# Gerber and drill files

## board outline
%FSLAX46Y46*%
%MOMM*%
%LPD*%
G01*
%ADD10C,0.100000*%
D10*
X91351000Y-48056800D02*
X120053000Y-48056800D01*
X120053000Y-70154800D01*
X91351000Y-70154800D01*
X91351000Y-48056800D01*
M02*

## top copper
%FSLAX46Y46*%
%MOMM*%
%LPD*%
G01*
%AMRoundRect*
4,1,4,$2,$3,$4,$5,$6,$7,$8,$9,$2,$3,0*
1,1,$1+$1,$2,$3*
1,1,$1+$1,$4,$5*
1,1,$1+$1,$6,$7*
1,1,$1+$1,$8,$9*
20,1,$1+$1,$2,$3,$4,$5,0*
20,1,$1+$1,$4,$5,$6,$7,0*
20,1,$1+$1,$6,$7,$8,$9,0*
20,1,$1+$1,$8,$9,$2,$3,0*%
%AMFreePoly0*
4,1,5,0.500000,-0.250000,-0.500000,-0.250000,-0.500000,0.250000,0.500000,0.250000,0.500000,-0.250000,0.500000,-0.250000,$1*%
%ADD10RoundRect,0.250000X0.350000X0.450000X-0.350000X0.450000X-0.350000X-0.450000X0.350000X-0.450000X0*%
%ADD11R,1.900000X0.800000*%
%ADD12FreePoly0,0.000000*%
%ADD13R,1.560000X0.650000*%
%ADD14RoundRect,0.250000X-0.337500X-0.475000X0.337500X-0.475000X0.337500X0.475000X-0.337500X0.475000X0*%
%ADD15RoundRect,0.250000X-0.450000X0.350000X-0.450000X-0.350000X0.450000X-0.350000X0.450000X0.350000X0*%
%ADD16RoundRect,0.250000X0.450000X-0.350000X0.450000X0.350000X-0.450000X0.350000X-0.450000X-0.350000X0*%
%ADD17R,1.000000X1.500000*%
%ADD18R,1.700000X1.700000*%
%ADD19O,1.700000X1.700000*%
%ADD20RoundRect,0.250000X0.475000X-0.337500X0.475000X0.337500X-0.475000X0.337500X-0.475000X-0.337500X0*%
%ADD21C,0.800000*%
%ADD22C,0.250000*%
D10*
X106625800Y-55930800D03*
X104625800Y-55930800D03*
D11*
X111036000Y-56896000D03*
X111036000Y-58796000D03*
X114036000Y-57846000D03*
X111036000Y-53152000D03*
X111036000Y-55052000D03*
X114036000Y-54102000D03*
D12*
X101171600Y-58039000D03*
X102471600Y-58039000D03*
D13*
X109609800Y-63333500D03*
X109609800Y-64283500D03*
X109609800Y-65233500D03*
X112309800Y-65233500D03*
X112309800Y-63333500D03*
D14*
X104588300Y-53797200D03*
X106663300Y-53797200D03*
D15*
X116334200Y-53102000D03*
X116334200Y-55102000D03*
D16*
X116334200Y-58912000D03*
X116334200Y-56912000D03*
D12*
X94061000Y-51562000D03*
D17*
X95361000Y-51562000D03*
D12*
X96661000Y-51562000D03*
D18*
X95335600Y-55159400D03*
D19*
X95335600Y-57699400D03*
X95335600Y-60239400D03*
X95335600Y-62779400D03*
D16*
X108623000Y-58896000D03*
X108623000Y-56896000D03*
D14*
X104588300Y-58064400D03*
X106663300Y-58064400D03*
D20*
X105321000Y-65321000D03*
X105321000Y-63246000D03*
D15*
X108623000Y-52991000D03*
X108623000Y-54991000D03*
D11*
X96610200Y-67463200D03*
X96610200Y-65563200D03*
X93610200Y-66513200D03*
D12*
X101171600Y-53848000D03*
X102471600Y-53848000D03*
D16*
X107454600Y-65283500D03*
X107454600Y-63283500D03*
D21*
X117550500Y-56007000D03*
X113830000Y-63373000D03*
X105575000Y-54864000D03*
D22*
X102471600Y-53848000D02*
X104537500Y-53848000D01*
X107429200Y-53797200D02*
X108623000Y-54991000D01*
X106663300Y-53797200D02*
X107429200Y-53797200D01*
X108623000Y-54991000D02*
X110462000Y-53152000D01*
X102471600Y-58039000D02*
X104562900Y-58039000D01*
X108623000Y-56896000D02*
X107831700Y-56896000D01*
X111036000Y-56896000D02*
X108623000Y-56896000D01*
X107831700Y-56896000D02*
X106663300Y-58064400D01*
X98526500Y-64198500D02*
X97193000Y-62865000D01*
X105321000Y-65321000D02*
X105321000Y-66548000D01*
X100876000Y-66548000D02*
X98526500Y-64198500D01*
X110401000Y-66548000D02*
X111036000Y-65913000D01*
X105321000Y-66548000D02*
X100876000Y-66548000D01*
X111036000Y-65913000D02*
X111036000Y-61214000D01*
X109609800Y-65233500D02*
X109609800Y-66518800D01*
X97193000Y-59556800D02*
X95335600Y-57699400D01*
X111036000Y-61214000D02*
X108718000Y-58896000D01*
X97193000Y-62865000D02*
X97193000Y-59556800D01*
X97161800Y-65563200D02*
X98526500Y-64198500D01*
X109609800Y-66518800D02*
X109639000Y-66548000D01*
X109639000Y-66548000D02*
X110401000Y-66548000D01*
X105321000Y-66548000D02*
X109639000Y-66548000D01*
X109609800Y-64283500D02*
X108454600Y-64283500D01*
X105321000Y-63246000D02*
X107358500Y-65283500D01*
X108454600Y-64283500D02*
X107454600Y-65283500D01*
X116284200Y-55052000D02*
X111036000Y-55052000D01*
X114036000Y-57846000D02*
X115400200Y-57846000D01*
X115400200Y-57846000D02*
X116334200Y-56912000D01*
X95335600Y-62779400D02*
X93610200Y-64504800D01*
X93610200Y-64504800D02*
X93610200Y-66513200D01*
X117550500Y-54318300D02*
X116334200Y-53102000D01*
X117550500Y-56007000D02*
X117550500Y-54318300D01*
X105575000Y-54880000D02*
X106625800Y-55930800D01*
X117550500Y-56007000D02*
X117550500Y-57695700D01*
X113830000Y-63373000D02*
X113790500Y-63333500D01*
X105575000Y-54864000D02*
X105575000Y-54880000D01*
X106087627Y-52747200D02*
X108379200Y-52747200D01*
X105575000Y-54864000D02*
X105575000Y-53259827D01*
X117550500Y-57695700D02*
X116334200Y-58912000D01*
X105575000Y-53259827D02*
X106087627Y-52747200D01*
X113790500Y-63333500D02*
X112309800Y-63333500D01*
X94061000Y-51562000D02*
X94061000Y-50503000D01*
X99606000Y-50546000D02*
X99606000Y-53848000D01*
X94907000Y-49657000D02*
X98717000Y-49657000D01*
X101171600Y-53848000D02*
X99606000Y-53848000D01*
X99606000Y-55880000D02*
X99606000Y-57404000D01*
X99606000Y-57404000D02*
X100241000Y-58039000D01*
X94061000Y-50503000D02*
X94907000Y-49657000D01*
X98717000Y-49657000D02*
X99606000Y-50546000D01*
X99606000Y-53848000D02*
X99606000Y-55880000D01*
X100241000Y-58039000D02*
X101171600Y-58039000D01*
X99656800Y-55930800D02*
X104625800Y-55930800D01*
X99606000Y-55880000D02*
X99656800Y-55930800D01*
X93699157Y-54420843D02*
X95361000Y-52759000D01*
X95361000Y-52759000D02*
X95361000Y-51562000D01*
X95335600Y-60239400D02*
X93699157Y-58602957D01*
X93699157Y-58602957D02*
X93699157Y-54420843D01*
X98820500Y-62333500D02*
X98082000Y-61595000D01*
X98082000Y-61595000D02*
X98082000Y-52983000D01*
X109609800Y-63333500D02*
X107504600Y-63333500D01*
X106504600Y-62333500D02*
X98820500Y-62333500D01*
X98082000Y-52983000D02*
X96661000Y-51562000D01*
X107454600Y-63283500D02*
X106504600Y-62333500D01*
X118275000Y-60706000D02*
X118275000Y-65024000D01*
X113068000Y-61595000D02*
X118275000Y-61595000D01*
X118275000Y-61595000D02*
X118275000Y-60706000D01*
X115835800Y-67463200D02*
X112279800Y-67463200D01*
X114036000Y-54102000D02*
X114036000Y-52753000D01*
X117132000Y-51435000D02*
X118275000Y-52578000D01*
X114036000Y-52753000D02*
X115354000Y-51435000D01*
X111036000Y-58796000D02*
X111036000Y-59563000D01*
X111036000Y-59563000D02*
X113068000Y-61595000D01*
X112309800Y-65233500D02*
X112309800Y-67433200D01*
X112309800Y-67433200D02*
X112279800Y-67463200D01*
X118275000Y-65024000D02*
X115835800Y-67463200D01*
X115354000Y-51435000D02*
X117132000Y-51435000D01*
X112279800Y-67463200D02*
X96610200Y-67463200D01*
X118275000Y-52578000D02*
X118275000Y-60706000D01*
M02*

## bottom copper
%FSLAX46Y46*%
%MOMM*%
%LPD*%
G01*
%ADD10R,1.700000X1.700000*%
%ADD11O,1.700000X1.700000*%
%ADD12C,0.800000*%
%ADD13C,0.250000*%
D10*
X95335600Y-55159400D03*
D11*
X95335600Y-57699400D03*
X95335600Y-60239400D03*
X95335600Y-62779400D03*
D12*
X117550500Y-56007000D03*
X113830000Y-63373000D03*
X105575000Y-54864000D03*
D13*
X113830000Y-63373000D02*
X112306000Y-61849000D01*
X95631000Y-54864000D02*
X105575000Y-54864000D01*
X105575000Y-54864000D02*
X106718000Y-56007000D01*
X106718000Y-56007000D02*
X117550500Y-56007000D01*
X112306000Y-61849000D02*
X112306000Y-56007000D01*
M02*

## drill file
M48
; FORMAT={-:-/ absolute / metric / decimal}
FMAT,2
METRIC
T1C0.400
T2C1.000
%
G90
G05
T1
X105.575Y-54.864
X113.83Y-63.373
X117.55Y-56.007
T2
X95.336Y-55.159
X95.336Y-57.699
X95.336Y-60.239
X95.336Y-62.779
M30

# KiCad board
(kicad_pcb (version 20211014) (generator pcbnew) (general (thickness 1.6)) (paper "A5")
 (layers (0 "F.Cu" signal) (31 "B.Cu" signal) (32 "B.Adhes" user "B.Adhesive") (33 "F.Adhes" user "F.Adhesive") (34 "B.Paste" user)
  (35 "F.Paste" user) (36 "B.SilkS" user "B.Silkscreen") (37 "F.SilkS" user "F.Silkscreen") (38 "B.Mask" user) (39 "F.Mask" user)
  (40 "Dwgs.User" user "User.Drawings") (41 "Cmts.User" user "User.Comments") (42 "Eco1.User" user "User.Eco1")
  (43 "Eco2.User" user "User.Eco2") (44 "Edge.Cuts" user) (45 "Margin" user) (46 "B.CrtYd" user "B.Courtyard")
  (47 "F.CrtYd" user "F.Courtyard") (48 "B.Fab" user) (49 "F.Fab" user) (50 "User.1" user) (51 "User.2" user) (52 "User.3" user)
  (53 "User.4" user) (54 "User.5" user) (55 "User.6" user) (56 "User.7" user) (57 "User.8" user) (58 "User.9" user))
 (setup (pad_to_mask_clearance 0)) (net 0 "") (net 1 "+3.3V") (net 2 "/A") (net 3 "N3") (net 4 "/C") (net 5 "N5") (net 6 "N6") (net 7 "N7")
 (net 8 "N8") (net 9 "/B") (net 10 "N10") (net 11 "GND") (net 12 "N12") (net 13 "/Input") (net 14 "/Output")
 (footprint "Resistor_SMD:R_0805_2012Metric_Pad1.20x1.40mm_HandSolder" (layer "F.Cu") (at 105.6258 55.9308 180)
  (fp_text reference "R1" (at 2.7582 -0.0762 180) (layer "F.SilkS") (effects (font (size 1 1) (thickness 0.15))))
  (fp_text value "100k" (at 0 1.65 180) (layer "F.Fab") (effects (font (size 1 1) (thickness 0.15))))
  (pad "1" smd roundrect (at -1 0 180) (size 1.2 1.4) (layers "F.Cu" "F.Paste" "F.Mask") (roundrect_rratio 0.2083333333) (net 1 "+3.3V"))
  (pad "2" smd roundrect (at 1 0 180) (size 1.2 1.4) (layers "F.Cu" "F.Paste" "F.Mask") (roundrect_rratio 0.2083333333) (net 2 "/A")))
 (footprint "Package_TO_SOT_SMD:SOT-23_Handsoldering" (layer "F.Cu") (at 112.536 57.846)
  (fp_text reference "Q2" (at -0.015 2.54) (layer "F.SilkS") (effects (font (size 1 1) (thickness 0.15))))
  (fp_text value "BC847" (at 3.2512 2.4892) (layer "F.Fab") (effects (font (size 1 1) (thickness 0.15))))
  (pad "1" smd rect (at -1.5 -0.95) (size 1.9 0.8) (layers "F.Cu" "F.Paste" "F.Mask") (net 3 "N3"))
  (pad "2" smd rect (at -1.5 0.95) (size 1.9 0.8) (layers "F.Cu" "F.Paste" "F.Mask") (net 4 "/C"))
  (pad "3" smd rect (at 1.5 0) (size 1.9 0.8) (layers "F.Cu" "F.Paste" "F.Mask") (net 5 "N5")))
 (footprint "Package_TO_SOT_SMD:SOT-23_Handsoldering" (layer "F.Cu") (at 112.536 54.102)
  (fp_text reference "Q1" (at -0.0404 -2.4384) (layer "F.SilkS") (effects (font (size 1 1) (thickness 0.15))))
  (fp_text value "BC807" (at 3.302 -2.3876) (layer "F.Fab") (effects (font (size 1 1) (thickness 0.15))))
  (pad "1" smd rect (at -1.5 -0.95) (size 1.9 0.8) (layers "F.Cu" "F.Paste" "F.Mask") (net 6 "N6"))
  (pad "2" smd rect (at -1.5 0.95) (size 1.9 0.8) (layers "F.Cu" "F.Paste" "F.Mask") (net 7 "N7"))
  (pad "3" smd rect (at 1.5 0) (size 1.9 0.8) (layers "F.Cu" "F.Paste" "F.Mask") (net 4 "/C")))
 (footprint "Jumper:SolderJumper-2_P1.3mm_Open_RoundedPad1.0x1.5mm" (layer "F.Cu") (at 101.8216 58.039)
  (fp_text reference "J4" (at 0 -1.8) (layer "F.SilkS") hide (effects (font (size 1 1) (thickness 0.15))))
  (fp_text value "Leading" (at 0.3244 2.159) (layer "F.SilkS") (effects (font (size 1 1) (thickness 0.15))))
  (pad "1" smd custom (at -0.65 0) (size 1 0.5) (layers "F.Cu" "F.Mask") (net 2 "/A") (zone_connect 2)
   (options (clearance outline) (anchor rect)) (primitives))
  (pad "2" smd custom (at 0.65 0) (size 1 0.5) (layers "F.Cu" "F.Mask") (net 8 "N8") (zone_connect 2)
   (options (clearance outline) (anchor rect)) (primitives)))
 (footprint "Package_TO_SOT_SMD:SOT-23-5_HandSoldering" (layer "F.Cu") (at 110.9598 64.2835)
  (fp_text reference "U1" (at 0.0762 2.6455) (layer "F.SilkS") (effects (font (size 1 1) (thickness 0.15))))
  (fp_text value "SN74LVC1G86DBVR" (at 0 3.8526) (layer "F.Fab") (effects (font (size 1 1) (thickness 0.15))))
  (pad "1" smd rect (at -1.35 -0.95) (size 1.56 0.65) (layers "F.Cu" "F.Paste" "F.Mask") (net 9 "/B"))
  (pad "2" smd rect (at -1.35 0) (size 1.56 0.65) (layers "F.Cu" "F.Paste" "F.Mask") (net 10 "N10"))
  (pad "3" smd rect (at -1.35 0.95) (size 1.56 0.65) (layers "F.Cu" "F.Paste" "F.Mask") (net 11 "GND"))
  (pad "4" smd rect (at 1.35 0.95) (size 1.56 0.65) (layers "F.Cu" "F.Paste" "F.Mask") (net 4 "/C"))
  (pad "5" smd rect (at 1.35 -0.95) (size 1.56 0.65) (layers "F.Cu" "F.Paste" "F.Mask") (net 1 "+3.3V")))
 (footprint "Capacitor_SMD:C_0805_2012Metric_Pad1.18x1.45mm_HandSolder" (layer "F.Cu") (at 105.6258 53.7972)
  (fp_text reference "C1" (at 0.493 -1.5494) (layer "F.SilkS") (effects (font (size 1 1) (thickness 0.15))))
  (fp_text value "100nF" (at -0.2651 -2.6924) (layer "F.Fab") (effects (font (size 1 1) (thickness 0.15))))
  (pad "1" smd roundrect (at -1.0375 0) (size 1.175 1.45) (layers "F.Cu" "F.Paste" "F.Mask") (roundrect_rratio 0.2127659574) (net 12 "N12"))
  (pad "2" smd roundrect (at 1.0375 0) (size 1.175 1.45) (layers "F.Cu" "F.Paste" "F.Mask") (roundrect_rratio 0.2127659574) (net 6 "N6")))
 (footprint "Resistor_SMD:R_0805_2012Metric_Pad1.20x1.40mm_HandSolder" (layer "F.Cu") (at 116.3342 54.102 -90)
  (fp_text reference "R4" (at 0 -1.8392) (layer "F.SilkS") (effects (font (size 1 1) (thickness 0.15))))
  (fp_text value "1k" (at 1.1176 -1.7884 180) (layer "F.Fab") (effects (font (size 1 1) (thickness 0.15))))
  (pad "1" smd roundrect (at -1 0 270) (size 1.2 1.4) (layers "F.Cu" "F.Paste" "F.Mask") (roundrect_rratio 0.2083333333) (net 1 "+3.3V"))
  (pad "2" smd roundrect (at 1 0 270) (size 1.2 1.4) (layers "F.Cu" "F.Paste" "F.Mask") (roundrect_rratio 0.2083333333) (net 7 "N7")))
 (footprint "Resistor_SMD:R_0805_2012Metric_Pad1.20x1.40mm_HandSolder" (layer "F.Cu") (at 116.3342 57.912 90)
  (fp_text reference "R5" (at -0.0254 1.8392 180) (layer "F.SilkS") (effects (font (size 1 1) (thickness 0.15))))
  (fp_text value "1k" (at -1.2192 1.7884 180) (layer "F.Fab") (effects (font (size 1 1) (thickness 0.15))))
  (pad "1" smd roundrect (at -1 0 90) (size 1.2 1.4) (layers "F.Cu" "F.Paste" "F.Mask") (roundrect_rratio 0.2083333333) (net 1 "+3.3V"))
  (pad "2" smd roundrect (at 1 0 90) (size 1.2 1.4) (layers "F.Cu" "F.Paste" "F.Mask") (roundrect_rratio 0.2083333333) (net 5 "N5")))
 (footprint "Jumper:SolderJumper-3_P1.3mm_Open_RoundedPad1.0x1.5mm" (layer "F.Cu") (at 95.361 51.562)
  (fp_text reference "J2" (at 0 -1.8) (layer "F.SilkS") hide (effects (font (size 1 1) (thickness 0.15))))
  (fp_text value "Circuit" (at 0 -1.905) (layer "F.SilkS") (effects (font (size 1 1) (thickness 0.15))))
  (pad "1" smd custom (at -1.3 0) (size 1 0.5) (layers "F.Cu" "F.Mask") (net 2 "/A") (zone_connect 2)
   (options (clearance outline) (anchor rect)) (primitives))
  (pad "2" smd rect (at 0 0) (size 1 1.5) (layers "F.Cu" "F.Mask") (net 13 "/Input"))
  (pad "3" smd custom (at 1.3 0) (size 1 0.5) (layers "F.Cu" "F.Mask") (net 9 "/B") (zone_connect 2)
   (options (clearance outline) (anchor rect)) (primitives)))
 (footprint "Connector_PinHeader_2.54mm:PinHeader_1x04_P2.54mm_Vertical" (layer "F.Cu") (at 95.3356 55.1594)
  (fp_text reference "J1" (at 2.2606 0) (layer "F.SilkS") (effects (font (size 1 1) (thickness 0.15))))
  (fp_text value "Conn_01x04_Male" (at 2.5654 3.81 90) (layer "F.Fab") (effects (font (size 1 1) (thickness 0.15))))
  (pad "1" thru_hole rect (at 0 0) (size 1.7 1.7) (drill 1) (layers *.Cu *.Mask) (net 1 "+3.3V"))
  (pad "2" thru_hole oval (at 0 2.54) (size 1.7 1.7) (drill 1) (layers *.Cu *.Mask) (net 11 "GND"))
  (pad "3" thru_hole oval (at 0 5.08) (size 1.7 1.7) (drill 1) (layers *.Cu *.Mask) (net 13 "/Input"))
  (pad "4" thru_hole oval (at 0 7.62) (size 1.7 1.7) (drill 1) (layers *.Cu *.Mask) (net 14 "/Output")))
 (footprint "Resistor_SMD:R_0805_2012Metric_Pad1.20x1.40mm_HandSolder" (layer "F.Cu") (at 108.623 57.896 90)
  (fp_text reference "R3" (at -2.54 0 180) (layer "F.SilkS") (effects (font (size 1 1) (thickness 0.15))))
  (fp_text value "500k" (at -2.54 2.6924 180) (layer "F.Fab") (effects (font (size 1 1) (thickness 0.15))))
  (pad "1" smd roundrect (at -1 0 90) (size 1.2 1.4) (layers "F.Cu" "F.Paste" "F.Mask") (roundrect_rratio 0.2083333333) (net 11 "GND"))
  (pad "2" smd roundrect (at 1 0 90) (size 1.2 1.4) (layers "F.Cu" "F.Paste" "F.Mask") (roundrect_rratio 0.2083333333) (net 3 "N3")))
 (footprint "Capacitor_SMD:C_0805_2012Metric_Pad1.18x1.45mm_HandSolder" (layer "F.Cu") (at 105.6258 58.0644)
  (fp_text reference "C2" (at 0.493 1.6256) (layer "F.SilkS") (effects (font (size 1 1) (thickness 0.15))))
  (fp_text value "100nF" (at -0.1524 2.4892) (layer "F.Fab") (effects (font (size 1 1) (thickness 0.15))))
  (pad "1" smd roundrect (at -1.0375 0) (size 1.175 1.45) (layers "F.Cu" "F.Paste" "F.Mask") (roundrect_rratio 0.2127659574) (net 8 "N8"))
  (pad "2" smd roundrect (at 1.0375 0) (size 1.175 1.45) (layers "F.Cu" "F.Paste" "F.Mask") (roundrect_rratio 0.2127659574) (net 3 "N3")))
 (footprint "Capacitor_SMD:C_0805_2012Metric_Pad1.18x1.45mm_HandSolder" (layer "F.Cu") (at 105.321 64.2835 90)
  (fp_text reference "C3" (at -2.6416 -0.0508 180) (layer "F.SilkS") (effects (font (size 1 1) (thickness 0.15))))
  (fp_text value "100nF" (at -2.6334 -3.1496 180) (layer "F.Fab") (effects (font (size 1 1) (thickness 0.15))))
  (pad "1" smd roundrect (at -1.0375 0 90) (size 1.175 1.45) (layers "F.Cu" "F.Paste" "F.Mask") (roundrect_rratio 0.2127659574)
   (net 11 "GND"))
  (pad "2" smd roundrect (at 1.0375 0 90) (size 1.175 1.45) (layers "F.Cu" "F.Paste" "F.Mask") (roundrect_rratio 0.2127659574)
   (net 10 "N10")))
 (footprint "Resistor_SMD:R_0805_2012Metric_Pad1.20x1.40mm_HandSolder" (layer "F.Cu") (at 108.623 53.991 -90)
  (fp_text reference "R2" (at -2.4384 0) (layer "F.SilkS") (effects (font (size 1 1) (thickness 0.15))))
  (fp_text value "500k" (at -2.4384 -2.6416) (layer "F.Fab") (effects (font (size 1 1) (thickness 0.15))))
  (pad "1" smd roundrect (at -1 0 270) (size 1.2 1.4) (layers "F.Cu" "F.Paste" "F.Mask") (roundrect_rratio 0.2083333333) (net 1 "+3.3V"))
  (pad "2" smd roundrect (at 1 0 270) (size 1.2 1.4) (layers "F.Cu" "F.Paste" "F.Mask") (roundrect_rratio 0.2083333333) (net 6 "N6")))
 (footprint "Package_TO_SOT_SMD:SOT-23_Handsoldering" (layer "F.Cu") (at 95.1102 66.5132 180)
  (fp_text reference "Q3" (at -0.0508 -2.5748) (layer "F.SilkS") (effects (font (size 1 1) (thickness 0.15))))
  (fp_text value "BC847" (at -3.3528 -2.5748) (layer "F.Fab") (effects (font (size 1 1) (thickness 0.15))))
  (pad "1" smd rect (at -1.5 -0.95 180) (size 1.9 0.8) (layers "F.Cu" "F.Paste" "F.Mask") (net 4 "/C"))
  (pad "2" smd rect (at -1.5 0.95 180) (size 1.9 0.8) (layers "F.Cu" "F.Paste" "F.Mask") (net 11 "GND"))
  (pad "3" smd rect (at 1.5 0 180) (size 1.9 0.8) (layers "F.Cu" "F.Paste" "F.Mask") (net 14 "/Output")))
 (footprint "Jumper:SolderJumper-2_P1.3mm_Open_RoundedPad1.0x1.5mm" (layer "F.Cu") (at 101.8216 53.848)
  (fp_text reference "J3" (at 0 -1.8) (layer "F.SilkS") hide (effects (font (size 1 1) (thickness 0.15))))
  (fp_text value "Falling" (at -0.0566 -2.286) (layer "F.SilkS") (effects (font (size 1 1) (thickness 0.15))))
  (pad "1" smd custom (at -0.65 0) (size 1 0.5) (layers "F.Cu" "F.Mask") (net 2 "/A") (zone_connect 2)
   (options (clearance outline) (anchor rect)) (primitives))
  (pad "2" smd custom (at 0.65 0) (size 1 0.5) (layers "F.Cu" "F.Mask") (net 12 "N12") (zone_connect 2)
   (options (clearance outline) (anchor rect)) (primitives)))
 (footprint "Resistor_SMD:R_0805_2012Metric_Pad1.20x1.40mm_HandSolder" (layer "F.Cu") (at 107.4546 64.2835 90)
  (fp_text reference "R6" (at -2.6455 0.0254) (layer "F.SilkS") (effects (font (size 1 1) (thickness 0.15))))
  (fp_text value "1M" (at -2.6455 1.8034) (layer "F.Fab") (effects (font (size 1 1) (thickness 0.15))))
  (pad "1" smd roundrect (at -1 0 90) (size 1.2 1.4) (layers "F.Cu" "F.Paste" "F.Mask") (roundrect_rratio 0.2083333333) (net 10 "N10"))
  (pad "2" smd roundrect (at 1 0 90) (size 1.2 1.4) (layers "F.Cu" "F.Paste" "F.Mask") (roundrect_rratio 0.2083333333) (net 9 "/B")))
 (gr_rect (start 120.053 70.1548) (end 91.351 48.0568) (layer "Edge.Cuts") (width 0.1) (fill none))
 (segment (start 102.4716 53.848) (end 104.5375 53.848) (width 0.25) (layer "F.Cu") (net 12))
 (segment (start 107.4292 53.7972) (end 108.623 54.991) (width 0.25) (layer "F.Cu") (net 6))
 (segment (start 106.6633 53.7972) (end 107.4292 53.7972) (width 0.25) (layer "F.Cu") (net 6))
 (segment (start 108.623 54.991) (end 110.462 53.152) (width 0.25) (layer "F.Cu") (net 6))
 (segment (start 102.4716 58.039) (end 104.5629 58.039) (width 0.25) (layer "F.Cu") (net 8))
 (segment (start 108.623 56.896) (end 107.8317 56.896) (width 0.25) (layer "F.Cu") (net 3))
 (segment (start 111.036 56.896) (end 108.623 56.896) (width 0.25) (layer "F.Cu") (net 3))
 (segment (start 107.8317 56.896) (end 106.6633 58.0644) (width 0.25) (layer "F.Cu") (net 3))
 (segment (start 98.5265 64.1985) (end 97.193 62.865) (width 0.25) (layer "F.Cu") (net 11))
 (segment (start 105.321 65.321) (end 105.321 66.548) (width 0.25) (layer "F.Cu") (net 11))
 (segment (start 100.876 66.548) (end 98.5265 64.1985) (width 0.25) (layer "F.Cu") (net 11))
 (segment (start 110.401 66.548) (end 111.036 65.913) (width 0.25) (layer "F.Cu") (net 11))
 (segment (start 105.321 66.548) (end 100.876 66.548) (width 0.25) (layer "F.Cu") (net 11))
 (segment (start 111.036 65.913) (end 111.036 61.214) (width 0.25) (layer "F.Cu") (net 11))
 (segment (start 109.6098 65.2335) (end 109.6098 66.5188) (width 0.25) (layer "F.Cu") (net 11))
 (segment (start 97.193 59.5568) (end 95.3356 57.6994) (width 0.25) (layer "F.Cu") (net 11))
 (segment (start 111.036 61.214) (end 108.718 58.896) (width 0.25) (layer "F.Cu") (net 11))
 (segment (start 97.193 62.865) (end 97.193 59.5568) (width 0.25) (layer "F.Cu") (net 11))
 (segment (start 97.1618 65.5632) (end 98.5265 64.1985) (width 0.25) (layer "F.Cu") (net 11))
 (segment (start 109.6098 66.5188) (end 109.639 66.548) (width 0.25) (layer "F.Cu") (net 11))
 (segment (start 109.639 66.548) (end 110.401 66.548) (width 0.25) (layer "F.Cu") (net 11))
 (segment (start 105.321 66.548) (end 109.639 66.548) (width 0.25) (layer "F.Cu") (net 11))
 (segment (start 109.6098 64.2835) (end 108.4546 64.2835) (width 0.25) (layer "F.Cu") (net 10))
 (segment (start 105.321 63.246) (end 107.3585 65.2835) (width 0.25) (layer "F.Cu") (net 10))
 (segment (start 108.4546 64.2835) (end 107.4546 65.2835) (width 0.25) (layer "F.Cu") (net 10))
 (segment (start 116.2842 55.052) (end 111.036 55.052) (width 0.25) (layer "F.Cu") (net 7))
 (segment (start 114.036 57.846) (end 115.4002 57.846) (width 0.25) (layer "F.Cu") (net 5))
 (segment (start 115.4002 57.846) (end 116.3342 56.912) (width 0.25) (layer "F.Cu") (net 5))
 (segment (start 95.3356 62.7794) (end 93.6102 64.5048) (width 0.25) (layer "F.Cu") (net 14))
 (segment (start 93.6102 64.5048) (end 93.6102 66.5132) (width 0.25) (layer "F.Cu") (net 14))
 (segment (start 117.5505 54.3183) (end 116.3342 53.102) (width 0.25) (layer "F.Cu") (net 1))
 (segment (start 117.5505 56.007) (end 117.5505 54.3183) (width 0.25) (layer "F.Cu") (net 1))
 (segment (start 105.575 54.88) (end 106.6258 55.9308) (width 0.25) (layer "F.Cu") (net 1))
 (segment (start 117.5505 56.007) (end 117.5505 57.6957) (width 0.25) (layer "F.Cu") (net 1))
 (segment (start 113.83 63.373) (end 113.7905 63.3335) (width 0.25) (layer "F.Cu") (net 1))
 (segment (start 105.575 54.864) (end 105.575 54.88) (width 0.25) (layer "F.Cu") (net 1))
 (segment (start 106.087627 52.7472) (end 108.3792 52.7472) (width 0.25) (layer "F.Cu") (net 1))
 (segment (start 105.575 54.864) (end 105.575 53.259827) (width 0.25) (layer "F.Cu") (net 1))
 (segment (start 117.5505 57.6957) (end 116.3342 58.912) (width 0.25) (layer "F.Cu") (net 1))
 (segment (start 105.575 53.259827) (end 106.087627 52.7472) (width 0.25) (layer "F.Cu") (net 1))
 (segment (start 113.7905 63.3335) (end 112.3098 63.3335) (width 0.25) (layer "F.Cu") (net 1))
 (via (at 117.5505 56.007) (size 0.8) (drill 0.4) (layers "F.Cu" "B.Cu") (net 1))
 (via (at 113.83 63.373) (size 0.8) (drill 0.4) (layers "F.Cu" "B.Cu") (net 1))
 (via (at 105.575 54.864) (size 0.8) (drill 0.4) (layers "F.Cu" "B.Cu") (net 1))
 (segment (start 113.83 63.373) (end 112.306 61.849) (width 0.25) (layer "B.Cu") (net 1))
 (segment (start 95.631 54.864) (end 105.575 54.864) (width 0.25) (layer "B.Cu") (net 1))
 (segment (start 105.575 54.864) (end 106.718 56.007) (width 0.25) (layer "B.Cu") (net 1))
 (segment (start 106.718 56.007) (end 117.5505 56.007) (width 0.25) (layer "B.Cu") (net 1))
 (segment (start 112.306 61.849) (end 112.306 56.007) (width 0.25) (layer "B.Cu") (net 1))
 (segment (start 94.061 51.562) (end 94.061 50.503) (width 0.25) (layer "F.Cu") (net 2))
 (segment (start 99.606 50.546) (end 99.606 53.848) (width 0.25) (layer "F.Cu") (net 2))
 (segment (start 94.907 49.657) (end 98.717 49.657) (width 0.25) (layer "F.Cu") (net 2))
 (segment (start 101.1716 53.848) (end 99.606 53.848) (width 0.25) (layer "F.Cu") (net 2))
 (segment (start 99.606 55.88) (end 99.606 57.404) (width 0.25) (layer "F.Cu") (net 2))
 (segment (start 99.606 57.404) (end 100.241 58.039) (width 0.25) (layer "F.Cu") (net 2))
 (segment (start 94.061 50.503) (end 94.907 49.657) (width 0.25) (layer "F.Cu") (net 2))
 (segment (start 98.717 49.657) (end 99.606 50.546) (width 0.25) (layer "F.Cu") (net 2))
 (segment (start 99.606 53.848) (end 99.606 55.88) (width 0.25) (layer "F.Cu") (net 2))
 (segment (start 100.241 58.039) (end 101.1716 58.039) (width 0.25) (layer "F.Cu") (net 2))
 (segment (start 99.6568 55.9308) (end 104.6258 55.9308) (width 0.25) (layer "F.Cu") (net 2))
 (segment (start 99.606 55.88) (end 99.6568 55.9308) (width 0.25) (layer "F.Cu") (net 2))
 (segment (start 93.699157 54.420843) (end 95.361 52.759) (width 0.25) (layer "F.Cu") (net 13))
 (segment (start 95.361 52.759) (end 95.361 51.562) (width 0.25) (layer "F.Cu") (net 13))
 (segment (start 95.3356 60.2394) (end 93.699157 58.602957) (width 0.25) (layer "F.Cu") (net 13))
 (segment (start 93.699157 58.602957) (end 93.699157 54.420843) (width 0.25) (layer "F.Cu") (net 13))
 (segment (start 98.8205 62.3335) (end 98.082 61.595) (width 0.25) (layer "F.Cu") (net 9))
 (segment (start 98.082 61.595) (end 98.082 52.983) (width 0.25) (layer "F.Cu") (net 9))
 (segment (start 109.6098 63.3335) (end 107.5046 63.3335) (width 0.25) (layer "F.Cu") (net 9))
 (segment (start 106.5046 62.3335) (end 98.8205 62.3335) (width 0.25) (layer "F.Cu") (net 9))
 (segment (start 98.082 52.983) (end 96.661 51.562) (width 0.25) (layer "F.Cu") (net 9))
 (segment (start 107.4546 63.2835) (end 106.5046 62.3335) (width 0.25) (layer "F.Cu") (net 9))
 (segment (start 118.275 60.706) (end 118.275 65.024) (width 0.25) (layer "F.Cu") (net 4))
 (segment (start 113.068 61.595) (end 118.275 61.595) (width 0.25) (layer "F.Cu") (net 4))
 (segment (start 118.275 61.595) (end 118.275 60.706) (width 0.25) (layer "F.Cu") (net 4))
 (segment (start 115.8358 67.4632) (end 112.2798 67.4632) (width 0.25) (layer "F.Cu") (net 4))
 (segment (start 114.036 54.102) (end 114.036 52.753) (width 0.25) (layer "F.Cu") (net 4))
 (segment (start 117.132 51.435) (end 118.275 52.578) (width 0.25) (layer "F.Cu") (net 4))
 (segment (start 114.036 52.753) (end 115.354 51.435) (width 0.25) (layer "F.Cu") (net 4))
 (segment (start 111.036 58.796) (end 111.036 59.563) (width 0.25) (layer "F.Cu") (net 4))
 (segment (start 111.036 59.563) (end 113.068 61.595) (width 0.25) (layer "F.Cu") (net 4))
 (segment (start 112.3098 65.2335) (end 112.3098 67.4332) (width 0.25) (layer "F.Cu") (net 4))
 (segment (start 112.3098 67.4332) (end 112.2798 67.4632) (width 0.25) (layer "F.Cu") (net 4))
 (segment (start 118.275 65.024) (end 115.8358 67.4632) (width 0.25) (layer "F.Cu") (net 4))
 (segment (start 115.354 51.435) (end 117.132 51.435) (width 0.25) (layer "F.Cu") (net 4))
 (segment (start 112.2798 67.4632) (end 96.6102 67.4632) (width 0.25) (layer "F.Cu") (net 4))
 (segment (start 118.275 52.578) (end 118.275 60.706) (width 0.25) (layer "F.Cu") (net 4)))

